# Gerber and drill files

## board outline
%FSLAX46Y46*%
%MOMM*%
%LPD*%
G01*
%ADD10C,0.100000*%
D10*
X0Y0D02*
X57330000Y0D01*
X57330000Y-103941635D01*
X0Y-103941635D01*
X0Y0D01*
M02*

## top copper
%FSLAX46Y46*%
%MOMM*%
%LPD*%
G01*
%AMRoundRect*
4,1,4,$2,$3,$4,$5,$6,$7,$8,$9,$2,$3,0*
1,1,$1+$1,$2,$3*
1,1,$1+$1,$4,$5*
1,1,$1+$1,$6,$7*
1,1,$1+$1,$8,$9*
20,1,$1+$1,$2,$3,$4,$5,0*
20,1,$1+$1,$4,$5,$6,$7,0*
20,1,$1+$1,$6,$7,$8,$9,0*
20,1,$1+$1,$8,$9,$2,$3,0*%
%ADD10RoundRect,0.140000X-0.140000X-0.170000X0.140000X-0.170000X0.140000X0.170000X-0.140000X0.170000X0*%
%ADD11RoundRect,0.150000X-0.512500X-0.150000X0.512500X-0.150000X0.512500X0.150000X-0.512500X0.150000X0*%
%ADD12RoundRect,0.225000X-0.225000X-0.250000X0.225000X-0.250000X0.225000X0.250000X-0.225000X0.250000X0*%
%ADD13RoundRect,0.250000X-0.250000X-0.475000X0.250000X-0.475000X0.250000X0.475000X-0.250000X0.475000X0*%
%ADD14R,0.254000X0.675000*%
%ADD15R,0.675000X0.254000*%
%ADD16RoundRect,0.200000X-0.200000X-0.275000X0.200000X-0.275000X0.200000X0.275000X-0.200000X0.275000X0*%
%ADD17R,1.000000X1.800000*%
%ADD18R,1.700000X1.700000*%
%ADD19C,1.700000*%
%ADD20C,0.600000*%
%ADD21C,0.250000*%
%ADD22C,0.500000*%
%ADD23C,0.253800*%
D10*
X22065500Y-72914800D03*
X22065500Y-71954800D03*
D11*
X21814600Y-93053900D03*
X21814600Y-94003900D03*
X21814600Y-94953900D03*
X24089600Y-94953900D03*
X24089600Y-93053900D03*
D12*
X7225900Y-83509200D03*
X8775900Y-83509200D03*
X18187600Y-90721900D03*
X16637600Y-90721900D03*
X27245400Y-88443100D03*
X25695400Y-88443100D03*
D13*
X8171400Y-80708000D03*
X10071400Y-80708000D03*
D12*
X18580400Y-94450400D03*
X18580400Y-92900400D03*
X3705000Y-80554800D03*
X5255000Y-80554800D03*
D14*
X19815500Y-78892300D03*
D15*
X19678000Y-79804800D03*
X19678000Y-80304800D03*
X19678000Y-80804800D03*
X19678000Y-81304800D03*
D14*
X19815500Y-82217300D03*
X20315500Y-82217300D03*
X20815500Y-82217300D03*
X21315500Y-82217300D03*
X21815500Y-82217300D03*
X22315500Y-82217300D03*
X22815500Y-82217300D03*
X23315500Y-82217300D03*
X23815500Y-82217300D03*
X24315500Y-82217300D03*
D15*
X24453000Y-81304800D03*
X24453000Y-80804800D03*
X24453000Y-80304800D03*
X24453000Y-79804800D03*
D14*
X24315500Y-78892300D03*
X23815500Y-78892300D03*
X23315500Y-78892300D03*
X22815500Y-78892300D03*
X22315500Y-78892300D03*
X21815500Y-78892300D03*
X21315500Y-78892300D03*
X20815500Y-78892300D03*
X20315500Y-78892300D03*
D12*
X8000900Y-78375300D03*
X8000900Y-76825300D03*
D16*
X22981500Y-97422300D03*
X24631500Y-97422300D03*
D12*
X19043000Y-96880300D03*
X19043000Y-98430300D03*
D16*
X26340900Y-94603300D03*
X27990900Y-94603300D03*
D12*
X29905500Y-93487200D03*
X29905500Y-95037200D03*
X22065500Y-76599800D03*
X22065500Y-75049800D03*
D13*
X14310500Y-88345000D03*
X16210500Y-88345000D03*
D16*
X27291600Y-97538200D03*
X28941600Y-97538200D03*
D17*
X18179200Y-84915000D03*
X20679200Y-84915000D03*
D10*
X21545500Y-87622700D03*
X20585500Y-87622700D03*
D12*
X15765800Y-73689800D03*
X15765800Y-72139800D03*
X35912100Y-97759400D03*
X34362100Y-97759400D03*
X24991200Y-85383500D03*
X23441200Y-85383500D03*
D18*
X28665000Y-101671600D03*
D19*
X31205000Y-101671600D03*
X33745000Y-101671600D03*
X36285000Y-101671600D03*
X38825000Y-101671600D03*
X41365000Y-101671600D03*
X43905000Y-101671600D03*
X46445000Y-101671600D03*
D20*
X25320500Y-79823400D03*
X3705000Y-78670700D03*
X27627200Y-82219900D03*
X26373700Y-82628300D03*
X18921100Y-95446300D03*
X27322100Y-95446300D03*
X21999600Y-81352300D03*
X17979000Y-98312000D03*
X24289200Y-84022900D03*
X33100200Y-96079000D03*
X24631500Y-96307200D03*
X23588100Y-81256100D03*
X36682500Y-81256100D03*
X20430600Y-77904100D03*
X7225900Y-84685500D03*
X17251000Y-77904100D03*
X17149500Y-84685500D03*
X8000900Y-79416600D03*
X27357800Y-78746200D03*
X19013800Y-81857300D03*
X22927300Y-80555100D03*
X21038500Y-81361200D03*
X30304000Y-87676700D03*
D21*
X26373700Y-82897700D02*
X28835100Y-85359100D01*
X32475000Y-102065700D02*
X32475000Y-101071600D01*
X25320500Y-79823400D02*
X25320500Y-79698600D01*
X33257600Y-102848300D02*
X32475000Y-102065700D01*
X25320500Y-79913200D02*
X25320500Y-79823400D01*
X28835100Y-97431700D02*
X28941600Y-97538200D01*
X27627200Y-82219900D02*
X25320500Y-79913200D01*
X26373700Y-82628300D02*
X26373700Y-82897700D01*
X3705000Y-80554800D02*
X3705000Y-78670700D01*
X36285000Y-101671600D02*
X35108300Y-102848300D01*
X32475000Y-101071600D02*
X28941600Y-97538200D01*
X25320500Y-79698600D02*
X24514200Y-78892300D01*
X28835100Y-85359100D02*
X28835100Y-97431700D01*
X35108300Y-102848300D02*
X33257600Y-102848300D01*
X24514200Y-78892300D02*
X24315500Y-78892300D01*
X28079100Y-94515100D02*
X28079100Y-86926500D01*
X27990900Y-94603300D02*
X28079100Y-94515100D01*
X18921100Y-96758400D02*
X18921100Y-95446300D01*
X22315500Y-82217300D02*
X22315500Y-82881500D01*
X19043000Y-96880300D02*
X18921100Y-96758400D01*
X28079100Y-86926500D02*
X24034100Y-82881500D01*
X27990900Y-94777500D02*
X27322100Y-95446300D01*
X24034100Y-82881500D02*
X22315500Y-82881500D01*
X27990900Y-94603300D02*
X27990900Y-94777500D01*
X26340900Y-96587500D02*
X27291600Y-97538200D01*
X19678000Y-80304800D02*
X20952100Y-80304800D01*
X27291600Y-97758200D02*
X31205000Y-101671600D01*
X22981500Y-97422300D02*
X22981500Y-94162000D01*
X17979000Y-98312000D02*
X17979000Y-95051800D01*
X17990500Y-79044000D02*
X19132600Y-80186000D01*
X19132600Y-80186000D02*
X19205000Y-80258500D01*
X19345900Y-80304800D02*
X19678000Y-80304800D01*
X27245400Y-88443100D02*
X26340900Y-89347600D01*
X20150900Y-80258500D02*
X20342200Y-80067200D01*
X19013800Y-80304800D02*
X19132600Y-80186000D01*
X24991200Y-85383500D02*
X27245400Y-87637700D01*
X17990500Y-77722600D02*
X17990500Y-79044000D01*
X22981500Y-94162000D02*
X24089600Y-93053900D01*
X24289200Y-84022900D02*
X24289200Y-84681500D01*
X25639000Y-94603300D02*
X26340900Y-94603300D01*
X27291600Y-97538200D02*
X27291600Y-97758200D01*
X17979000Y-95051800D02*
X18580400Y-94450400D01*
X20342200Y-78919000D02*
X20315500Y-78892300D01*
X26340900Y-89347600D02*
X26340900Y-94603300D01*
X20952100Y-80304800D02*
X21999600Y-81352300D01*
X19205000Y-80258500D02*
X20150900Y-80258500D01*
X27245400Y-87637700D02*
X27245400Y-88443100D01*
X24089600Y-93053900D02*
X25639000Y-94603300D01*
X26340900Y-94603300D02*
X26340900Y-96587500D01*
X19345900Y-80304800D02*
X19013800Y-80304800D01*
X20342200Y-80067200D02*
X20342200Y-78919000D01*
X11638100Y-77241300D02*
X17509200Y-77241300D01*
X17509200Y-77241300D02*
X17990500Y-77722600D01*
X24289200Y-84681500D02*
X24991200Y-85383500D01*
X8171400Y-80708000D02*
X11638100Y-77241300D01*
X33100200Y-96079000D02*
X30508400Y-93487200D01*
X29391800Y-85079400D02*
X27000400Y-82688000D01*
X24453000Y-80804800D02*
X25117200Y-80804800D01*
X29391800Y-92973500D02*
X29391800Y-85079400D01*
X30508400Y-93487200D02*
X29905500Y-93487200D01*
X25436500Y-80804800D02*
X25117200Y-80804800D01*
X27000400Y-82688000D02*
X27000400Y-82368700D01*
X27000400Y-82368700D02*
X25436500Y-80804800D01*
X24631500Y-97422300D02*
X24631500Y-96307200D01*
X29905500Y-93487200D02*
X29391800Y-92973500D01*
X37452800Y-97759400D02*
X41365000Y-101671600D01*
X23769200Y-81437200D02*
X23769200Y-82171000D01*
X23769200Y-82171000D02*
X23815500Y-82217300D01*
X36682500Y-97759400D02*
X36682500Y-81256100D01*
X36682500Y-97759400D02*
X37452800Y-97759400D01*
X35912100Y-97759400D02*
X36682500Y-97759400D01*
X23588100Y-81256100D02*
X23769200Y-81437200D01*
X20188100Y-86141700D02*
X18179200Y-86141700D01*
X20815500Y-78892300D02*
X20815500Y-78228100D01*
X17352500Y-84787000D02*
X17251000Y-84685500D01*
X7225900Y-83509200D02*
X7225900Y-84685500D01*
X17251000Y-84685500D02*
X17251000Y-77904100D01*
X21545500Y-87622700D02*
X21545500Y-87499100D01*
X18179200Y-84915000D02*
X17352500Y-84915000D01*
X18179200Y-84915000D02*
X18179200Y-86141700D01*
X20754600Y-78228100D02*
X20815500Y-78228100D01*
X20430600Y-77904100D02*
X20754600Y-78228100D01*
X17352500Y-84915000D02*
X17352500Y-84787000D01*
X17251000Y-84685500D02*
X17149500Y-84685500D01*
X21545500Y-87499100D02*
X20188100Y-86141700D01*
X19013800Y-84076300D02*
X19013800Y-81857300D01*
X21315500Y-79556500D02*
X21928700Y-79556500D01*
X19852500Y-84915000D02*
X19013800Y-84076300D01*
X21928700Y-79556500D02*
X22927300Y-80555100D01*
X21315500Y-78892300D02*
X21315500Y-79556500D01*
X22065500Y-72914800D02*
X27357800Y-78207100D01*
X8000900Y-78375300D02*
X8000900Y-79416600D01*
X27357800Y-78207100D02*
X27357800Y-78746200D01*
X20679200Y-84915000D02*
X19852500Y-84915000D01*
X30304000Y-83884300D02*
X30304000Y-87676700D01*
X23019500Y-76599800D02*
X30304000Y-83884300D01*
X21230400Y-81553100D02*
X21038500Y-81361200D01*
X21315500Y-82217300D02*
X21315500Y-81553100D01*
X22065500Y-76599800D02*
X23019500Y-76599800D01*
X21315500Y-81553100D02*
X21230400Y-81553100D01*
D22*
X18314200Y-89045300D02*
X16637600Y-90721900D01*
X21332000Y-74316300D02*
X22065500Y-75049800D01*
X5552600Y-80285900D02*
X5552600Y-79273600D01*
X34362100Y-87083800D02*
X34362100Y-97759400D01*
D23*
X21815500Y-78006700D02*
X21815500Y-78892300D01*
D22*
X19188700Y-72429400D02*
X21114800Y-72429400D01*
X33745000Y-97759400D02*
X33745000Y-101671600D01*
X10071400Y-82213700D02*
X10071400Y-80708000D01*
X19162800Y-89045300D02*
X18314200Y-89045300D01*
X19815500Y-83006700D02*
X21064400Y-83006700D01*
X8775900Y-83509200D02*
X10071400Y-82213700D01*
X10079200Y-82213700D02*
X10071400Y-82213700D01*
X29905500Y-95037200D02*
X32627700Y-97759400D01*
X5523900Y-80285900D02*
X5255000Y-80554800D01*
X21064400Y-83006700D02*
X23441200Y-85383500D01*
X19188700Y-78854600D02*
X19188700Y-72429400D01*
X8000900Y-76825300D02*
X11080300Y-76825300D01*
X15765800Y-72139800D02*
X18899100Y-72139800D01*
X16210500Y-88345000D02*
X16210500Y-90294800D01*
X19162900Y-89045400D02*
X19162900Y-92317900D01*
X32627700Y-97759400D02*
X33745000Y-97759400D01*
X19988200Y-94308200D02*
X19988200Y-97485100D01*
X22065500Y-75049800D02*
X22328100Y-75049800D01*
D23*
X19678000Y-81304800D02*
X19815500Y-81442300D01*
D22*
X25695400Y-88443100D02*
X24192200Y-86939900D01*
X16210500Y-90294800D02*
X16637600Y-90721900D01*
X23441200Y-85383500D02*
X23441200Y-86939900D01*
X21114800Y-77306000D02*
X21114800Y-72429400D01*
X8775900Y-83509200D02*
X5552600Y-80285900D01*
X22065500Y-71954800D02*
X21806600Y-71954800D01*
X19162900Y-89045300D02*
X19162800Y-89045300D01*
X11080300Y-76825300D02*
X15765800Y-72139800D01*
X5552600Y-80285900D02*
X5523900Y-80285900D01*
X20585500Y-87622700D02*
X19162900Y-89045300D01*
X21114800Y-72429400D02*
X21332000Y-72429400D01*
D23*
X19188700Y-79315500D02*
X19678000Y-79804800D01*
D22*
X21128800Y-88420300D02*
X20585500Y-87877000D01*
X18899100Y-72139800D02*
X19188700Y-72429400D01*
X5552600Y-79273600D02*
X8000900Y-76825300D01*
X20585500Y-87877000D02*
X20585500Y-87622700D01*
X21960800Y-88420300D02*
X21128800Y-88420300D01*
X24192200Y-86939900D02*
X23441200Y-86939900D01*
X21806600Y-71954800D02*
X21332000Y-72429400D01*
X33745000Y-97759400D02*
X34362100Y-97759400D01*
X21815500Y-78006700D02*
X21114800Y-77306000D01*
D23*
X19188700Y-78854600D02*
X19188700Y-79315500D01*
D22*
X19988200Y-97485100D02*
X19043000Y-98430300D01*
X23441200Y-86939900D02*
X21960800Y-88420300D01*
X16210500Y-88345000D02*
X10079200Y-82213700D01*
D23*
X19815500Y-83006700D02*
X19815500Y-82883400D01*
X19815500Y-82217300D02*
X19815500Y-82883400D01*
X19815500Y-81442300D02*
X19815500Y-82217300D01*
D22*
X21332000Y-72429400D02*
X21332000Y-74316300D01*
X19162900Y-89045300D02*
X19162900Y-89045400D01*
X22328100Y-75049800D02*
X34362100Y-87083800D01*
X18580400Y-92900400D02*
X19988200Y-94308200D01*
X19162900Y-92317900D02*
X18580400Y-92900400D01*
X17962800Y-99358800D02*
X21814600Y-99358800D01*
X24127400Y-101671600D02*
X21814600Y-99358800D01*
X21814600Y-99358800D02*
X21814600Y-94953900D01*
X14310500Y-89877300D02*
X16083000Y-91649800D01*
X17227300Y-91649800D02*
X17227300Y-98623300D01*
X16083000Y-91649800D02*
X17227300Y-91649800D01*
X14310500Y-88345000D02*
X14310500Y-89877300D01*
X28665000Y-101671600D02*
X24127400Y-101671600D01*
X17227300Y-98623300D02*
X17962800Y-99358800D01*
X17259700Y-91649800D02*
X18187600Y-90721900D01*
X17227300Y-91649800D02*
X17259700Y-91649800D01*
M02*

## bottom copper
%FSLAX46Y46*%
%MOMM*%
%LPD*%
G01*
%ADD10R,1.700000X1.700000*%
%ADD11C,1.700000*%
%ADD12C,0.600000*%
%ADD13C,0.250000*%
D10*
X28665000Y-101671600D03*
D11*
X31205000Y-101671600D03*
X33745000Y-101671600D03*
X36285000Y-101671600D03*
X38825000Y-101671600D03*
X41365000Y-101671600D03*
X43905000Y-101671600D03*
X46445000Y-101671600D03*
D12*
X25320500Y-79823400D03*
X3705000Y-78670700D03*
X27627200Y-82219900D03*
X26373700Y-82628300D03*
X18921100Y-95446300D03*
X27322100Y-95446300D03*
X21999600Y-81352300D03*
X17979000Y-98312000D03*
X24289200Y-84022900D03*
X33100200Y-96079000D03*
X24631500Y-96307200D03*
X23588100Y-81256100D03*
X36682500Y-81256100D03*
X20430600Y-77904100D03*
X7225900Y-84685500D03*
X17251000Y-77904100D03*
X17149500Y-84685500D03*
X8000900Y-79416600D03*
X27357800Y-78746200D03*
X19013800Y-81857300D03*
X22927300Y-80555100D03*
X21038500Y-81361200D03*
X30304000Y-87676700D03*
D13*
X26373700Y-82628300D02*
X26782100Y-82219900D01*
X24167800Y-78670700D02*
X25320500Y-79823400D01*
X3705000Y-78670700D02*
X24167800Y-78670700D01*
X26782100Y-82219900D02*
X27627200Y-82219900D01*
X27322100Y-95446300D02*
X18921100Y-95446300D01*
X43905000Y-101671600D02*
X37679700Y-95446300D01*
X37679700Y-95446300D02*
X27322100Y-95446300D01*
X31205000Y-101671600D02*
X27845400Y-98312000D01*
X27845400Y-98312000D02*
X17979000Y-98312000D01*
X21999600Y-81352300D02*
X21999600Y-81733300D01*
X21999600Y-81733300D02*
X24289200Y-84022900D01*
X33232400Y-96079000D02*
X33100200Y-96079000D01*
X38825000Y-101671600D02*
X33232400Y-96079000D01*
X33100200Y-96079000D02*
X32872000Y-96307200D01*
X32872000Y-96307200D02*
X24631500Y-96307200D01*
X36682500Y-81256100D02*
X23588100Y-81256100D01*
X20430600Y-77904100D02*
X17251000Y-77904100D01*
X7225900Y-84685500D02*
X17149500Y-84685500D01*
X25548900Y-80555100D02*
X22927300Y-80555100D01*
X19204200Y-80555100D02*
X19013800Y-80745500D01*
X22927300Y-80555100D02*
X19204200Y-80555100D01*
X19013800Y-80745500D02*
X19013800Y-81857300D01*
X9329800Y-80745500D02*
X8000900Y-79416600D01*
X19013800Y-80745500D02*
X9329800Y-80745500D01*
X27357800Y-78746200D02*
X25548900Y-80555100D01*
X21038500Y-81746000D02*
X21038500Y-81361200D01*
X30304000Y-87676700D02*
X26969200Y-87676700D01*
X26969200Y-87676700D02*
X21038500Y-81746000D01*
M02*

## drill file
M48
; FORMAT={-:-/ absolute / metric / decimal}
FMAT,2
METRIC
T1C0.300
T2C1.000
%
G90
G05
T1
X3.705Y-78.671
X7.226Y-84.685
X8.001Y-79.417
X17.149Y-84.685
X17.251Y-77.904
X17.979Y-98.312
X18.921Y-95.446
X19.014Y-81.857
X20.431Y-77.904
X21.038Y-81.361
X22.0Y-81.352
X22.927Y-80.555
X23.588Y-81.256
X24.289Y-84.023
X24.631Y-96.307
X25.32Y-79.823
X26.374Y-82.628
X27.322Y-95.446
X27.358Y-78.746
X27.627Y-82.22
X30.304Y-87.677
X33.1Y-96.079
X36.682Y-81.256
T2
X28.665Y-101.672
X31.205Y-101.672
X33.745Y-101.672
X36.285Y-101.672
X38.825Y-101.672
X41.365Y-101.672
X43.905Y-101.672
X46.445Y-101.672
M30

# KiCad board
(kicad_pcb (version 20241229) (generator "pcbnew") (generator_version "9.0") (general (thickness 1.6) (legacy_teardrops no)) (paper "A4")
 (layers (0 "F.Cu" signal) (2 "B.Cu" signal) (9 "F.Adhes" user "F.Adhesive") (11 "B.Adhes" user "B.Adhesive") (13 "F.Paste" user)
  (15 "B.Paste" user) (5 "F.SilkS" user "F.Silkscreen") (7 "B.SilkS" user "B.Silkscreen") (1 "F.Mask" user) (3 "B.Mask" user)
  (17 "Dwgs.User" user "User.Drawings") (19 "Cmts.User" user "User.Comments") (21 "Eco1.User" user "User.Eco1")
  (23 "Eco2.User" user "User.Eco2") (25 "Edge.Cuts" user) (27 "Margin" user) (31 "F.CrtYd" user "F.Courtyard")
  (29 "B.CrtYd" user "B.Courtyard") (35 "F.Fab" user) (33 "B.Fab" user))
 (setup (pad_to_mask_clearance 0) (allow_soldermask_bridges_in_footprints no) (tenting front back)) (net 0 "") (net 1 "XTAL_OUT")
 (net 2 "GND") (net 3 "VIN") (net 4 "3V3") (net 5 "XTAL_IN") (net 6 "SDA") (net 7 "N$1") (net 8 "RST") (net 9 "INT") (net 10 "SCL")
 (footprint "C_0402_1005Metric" (layer "F.Cu") (at 22.0655 72.4348 90)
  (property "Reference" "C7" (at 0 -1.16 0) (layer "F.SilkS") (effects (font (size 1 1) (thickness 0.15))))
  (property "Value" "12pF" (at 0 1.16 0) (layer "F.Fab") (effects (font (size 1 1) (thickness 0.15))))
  (pad "1" smd roundrect (at -0.48 0) (size 0.56 0.62) (layers "F.Cu" "F.Mask" "F.Paste") (roundrect_rratio 0.25) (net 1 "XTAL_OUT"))
  (pad "2" smd roundrect (at 0.48 0) (size 0.56 0.62) (layers "F.Cu" "F.Mask" "F.Paste") (roundrect_rratio 0.25) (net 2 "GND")))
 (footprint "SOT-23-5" (layer "F.Cu") (at 22.9521 94.0039)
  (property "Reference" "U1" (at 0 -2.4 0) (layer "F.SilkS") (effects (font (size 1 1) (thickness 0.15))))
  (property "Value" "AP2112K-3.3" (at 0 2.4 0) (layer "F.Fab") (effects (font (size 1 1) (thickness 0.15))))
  (pad "1" smd roundrect (at -1.1375 -0.95) (size 1.325 0.6) (layers "F.Cu" "F.Mask" "F.Paste") (roundrect_rratio 0.25) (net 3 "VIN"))
  (pad "2" smd roundrect (at -1.1375 0) (size 1.325 0.6) (layers "F.Cu" "F.Mask" "F.Paste") (roundrect_rratio 0.25) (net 2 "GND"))
  (pad "3" smd roundrect (at -1.1375 0.95) (size 1.325 0.6) (layers "F.Cu" "F.Mask" "F.Paste") (roundrect_rratio 0.25) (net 3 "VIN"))
  (pad "4" smd roundrect (at 1.1375 0.95) (size 1.325 0.6) (layers "F.Cu" "F.Mask" "F.Paste") (roundrect_rratio 0.25))
  (pad "5" smd roundrect (at 1.1375 -0.95) (size 1.325 0.6) (layers "F.Cu" "F.Mask" "F.Paste") (roundrect_rratio 0.25) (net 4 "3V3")))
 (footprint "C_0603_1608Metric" (layer "F.Cu") (at 8.0009 83.5092)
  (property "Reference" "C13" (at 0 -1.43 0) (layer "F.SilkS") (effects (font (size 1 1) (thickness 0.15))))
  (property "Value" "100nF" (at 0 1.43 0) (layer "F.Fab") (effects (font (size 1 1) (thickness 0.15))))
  (pad "1" smd roundrect (at -0.775 0) (size 0.9 0.95) (layers "F.Cu" "F.Mask" "F.Paste") (roundrect_rratio 0.25) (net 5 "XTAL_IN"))
  (pad "2" smd roundrect (at 0.775 0) (size 0.9 0.95) (layers "F.Cu" "F.Mask" "F.Paste") (roundrect_rratio 0.25) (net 2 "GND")))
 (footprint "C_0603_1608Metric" (layer "F.Cu") (at 17.4126 90.7219 180)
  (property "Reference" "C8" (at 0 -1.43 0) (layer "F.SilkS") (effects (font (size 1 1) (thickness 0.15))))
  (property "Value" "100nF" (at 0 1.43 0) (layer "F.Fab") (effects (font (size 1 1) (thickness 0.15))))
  (pad "1" smd roundrect (at -0.775 0) (size 0.9 0.95) (layers "F.Cu" "F.Mask" "F.Paste") (roundrect_rratio 0.25) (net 3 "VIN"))
  (pad "2" smd roundrect (at 0.775 0) (size 0.9 0.95) (layers "F.Cu" "F.Mask" "F.Paste") (roundrect_rratio 0.25) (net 2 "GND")))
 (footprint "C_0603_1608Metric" (layer "F.Cu") (at 26.4704 88.4431 180)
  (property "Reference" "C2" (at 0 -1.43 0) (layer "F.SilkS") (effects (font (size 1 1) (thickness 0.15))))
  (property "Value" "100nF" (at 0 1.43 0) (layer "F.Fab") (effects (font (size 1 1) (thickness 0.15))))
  (pad "1" smd roundrect (at -0.775 0) (size 0.9 0.95) (layers "F.Cu" "F.Mask" "F.Paste") (roundrect_rratio 0.25) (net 4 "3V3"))
  (pad "2" smd roundrect (at 0.775 0) (size 0.9 0.95) (layers "F.Cu" "F.Mask" "F.Paste") (roundrect_rratio 0.25) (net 2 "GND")))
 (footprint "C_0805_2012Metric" (layer "F.Cu") (at 9.1214 80.708)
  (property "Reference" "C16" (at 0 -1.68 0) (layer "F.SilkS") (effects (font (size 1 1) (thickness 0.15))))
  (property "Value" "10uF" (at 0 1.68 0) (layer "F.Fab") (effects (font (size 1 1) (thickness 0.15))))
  (pad "1" smd roundrect (at -0.95 0) (size 1 1.45) (layers "F.Cu" "F.Mask" "F.Paste") (roundrect_rratio 0.25) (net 4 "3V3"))
  (pad "2" smd roundrect (at 0.95 0) (size 1 1.45) (layers "F.Cu" "F.Mask" "F.Paste") (roundrect_rratio 0.25) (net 2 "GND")))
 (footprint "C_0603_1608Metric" (layer "F.Cu") (at 18.5804 93.6754 90)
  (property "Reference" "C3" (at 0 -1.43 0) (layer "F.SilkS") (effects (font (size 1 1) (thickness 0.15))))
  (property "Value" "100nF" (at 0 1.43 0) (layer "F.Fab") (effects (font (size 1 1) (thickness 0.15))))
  (pad "1" smd roundrect (at -0.775 0) (size 0.9 0.95) (layers "F.Cu" "F.Mask" "F.Paste") (roundrect_rratio 0.25) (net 4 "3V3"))
  (pad "2" smd roundrect (at 0.775 0) (size 0.9 0.95) (layers "F.Cu" "F.Mask" "F.Paste") (roundrect_rratio 0.25) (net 2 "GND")))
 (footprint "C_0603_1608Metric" (layer "F.Cu") (at 4.48 80.5548)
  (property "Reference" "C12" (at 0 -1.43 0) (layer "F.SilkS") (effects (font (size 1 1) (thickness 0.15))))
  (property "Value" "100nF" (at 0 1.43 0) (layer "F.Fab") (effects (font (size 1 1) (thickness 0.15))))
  (pad "1" smd roundrect (at -0.775 0) (size 0.9 0.95) (layers "F.Cu" "F.Mask" "F.Paste") (roundrect_rratio 0.25) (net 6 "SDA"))
  (pad "2" smd roundrect (at 0.775 0) (size 0.9 0.95) (layers "F.Cu" "F.Mask" "F.Paste") (roundrect_rratio 0.25) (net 2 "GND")))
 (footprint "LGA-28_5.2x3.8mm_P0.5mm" (layer "F.Cu") (at 22.0655 80.5548)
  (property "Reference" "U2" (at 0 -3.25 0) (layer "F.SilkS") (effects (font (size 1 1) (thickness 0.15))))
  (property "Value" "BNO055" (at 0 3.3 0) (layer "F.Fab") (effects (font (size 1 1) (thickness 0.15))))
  (pad "1" smd rect (at -2.25 -1.6625) (size 0.254 0.675) (layers "F.Cu" "F.Mask" "F.Paste"))
  (pad "2" smd rect (at -2.3875 -0.75 90) (size 0.254 0.675) (layers "F.Cu" "F.Mask" "F.Paste") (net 2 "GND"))
  (pad "3" smd rect (at -2.3875 -0.25 90) (size 0.254 0.675) (layers "F.Cu" "F.Mask" "F.Paste") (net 4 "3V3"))
  (pad "4" smd rect (at -2.3875 0.25 90) (size 0.254 0.675) (layers "F.Cu" "F.Mask" "F.Paste"))
  (pad "5" smd rect (at -2.3875 0.75 90) (size 0.254 0.675) (layers "F.Cu" "F.Mask" "F.Paste") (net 2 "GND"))
  (pad "6" smd rect (at -2.25 1.6625) (size 0.254 0.675) (layers "F.Cu" "F.Mask" "F.Paste") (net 2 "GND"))
  (pad "7" smd rect (at -1.75 1.6625) (size 0.254 0.675) (layers "F.Cu" "F.Mask" "F.Paste"))
  (pad "8" smd rect (at -1.25 1.6625) (size 0.254 0.675) (layers "F.Cu" "F.Mask" "F.Paste"))
  (pad "9" smd rect (at -0.75 1.6625) (size 0.254 0.675) (layers "F.Cu" "F.Mask" "F.Paste") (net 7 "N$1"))
  (pad "10" smd rect (at -0.25 1.6625) (size 0.254 0.675) (layers "F.Cu" "F.Mask" "F.Paste"))
  (pad "11" smd rect (at 0.25 1.6625) (size 0.254 0.675) (layers "F.Cu" "F.Mask" "F.Paste") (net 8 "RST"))
  (pad "12" smd rect (at 0.75 1.6625) (size 0.254 0.675) (layers "F.Cu" "F.Mask" "F.Paste"))
  (pad "13" smd rect (at 1.25 1.6625) (size 0.254 0.675) (layers "F.Cu" "F.Mask" "F.Paste"))
  (pad "14" smd rect (at 1.75 1.6625) (size 0.254 0.675) (layers "F.Cu" "F.Mask" "F.Paste") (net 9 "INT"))
  (pad "15" smd rect (at 2.25 1.6625) (size 0.254 0.675) (layers "F.Cu" "F.Mask" "F.Paste"))
  (pad "16" smd rect (at 2.3875 0.75 90) (size 0.254 0.675) (layers "F.Cu" "F.Mask" "F.Paste"))
  (pad "17" smd rect (at 2.3875 0.25 90) (size 0.254 0.675) (layers "F.Cu" "F.Mask" "F.Paste") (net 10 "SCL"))
  (pad "18" smd rect (at 2.3875 -0.25 90) (size 0.254 0.675) (layers "F.Cu" "F.Mask" "F.Paste"))
  (pad "19" smd rect (at 2.3875 -0.75 90) (size 0.254 0.675) (layers "F.Cu" "F.Mask" "F.Paste"))
  (pad "20" smd rect (at 2.25 -1.6625) (size 0.254 0.675) (layers "F.Cu" "F.Mask" "F.Paste") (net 6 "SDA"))
  (pad "21" smd rect (at 1.75 -1.6625) (size 0.254 0.675) (layers "F.Cu" "F.Mask" "F.Paste"))
  (pad "22" smd rect (at 1.25 -1.6625) (size 0.254 0.675) (layers "F.Cu" "F.Mask" "F.Paste"))
  (pad "23" smd rect (at 0.75 -1.6625) (size 0.254 0.675) (layers "F.Cu" "F.Mask" "F.Paste"))
  (pad "24" smd rect (at 0.25 -1.6625) (size 0.254 0.675) (layers "F.Cu" "F.Mask" "F.Paste"))
  (pad "25" smd rect (at -0.25 -1.6625) (size 0.254 0.675) (layers "F.Cu" "F.Mask" "F.Paste") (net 2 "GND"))
  (pad "26" smd rect (at -0.75 -1.6625) (size 0.254 0.675) (layers "F.Cu" "F.Mask" "F.Paste") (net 1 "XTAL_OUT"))
  (pad "27" smd rect (at -1.25 -1.6625) (size 0.254 0.675) (layers "F.Cu" "F.Mask" "F.Paste") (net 5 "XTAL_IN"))
  (pad "28" smd rect (at -1.75 -1.6625) (size 0.254 0.675) (layers "F.Cu" "F.Mask" "F.Paste") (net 4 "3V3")))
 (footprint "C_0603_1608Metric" (layer "F.Cu") (at 8.0009 77.6003 90)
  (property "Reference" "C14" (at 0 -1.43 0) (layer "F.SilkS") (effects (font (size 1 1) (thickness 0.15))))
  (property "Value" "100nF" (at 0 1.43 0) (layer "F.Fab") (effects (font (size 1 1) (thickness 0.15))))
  (pad "1" smd roundrect (at -0.775 0) (size 0.9 0.95) (layers "F.Cu" "F.Mask" "F.Paste") (roundrect_rratio 0.25) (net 1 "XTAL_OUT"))
  (pad "2" smd roundrect (at 0.775 0) (size 0.9 0.95) (layers "F.Cu" "F.Mask" "F.Paste") (roundrect_rratio 0.25) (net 2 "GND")))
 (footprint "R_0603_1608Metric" (layer "F.Cu") (at 23.8065 97.4223)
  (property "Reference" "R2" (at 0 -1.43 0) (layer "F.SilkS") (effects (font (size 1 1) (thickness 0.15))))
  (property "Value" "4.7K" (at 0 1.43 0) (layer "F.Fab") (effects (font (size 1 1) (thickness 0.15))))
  (pad "1" smd roundrect (at -0.825 0) (size 0.8 0.95) (layers "F.Cu" "F.Mask" "F.Paste") (roundrect_rratio 0.25) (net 4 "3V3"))
  (pad "2" smd roundrect (at 0.825 0) (size 0.8 0.95) (layers "F.Cu" "F.Mask" "F.Paste") (roundrect_rratio 0.25) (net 10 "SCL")))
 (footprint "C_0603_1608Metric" (layer "F.Cu") (at 19.043 97.6553 -90)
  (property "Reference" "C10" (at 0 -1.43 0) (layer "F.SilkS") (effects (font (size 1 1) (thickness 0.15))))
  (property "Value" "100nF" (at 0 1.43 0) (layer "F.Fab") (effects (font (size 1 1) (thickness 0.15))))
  (pad "1" smd roundrect (at -0.775 0) (size 0.9 0.95) (layers "F.Cu" "F.Mask" "F.Paste") (roundrect_rratio 0.25) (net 8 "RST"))
  (pad "2" smd roundrect (at 0.775 0) (size 0.9 0.95) (layers "F.Cu" "F.Mask" "F.Paste") (roundrect_rratio 0.25) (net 2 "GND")))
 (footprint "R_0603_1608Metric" (layer "F.Cu") (at 27.1659 94.6033)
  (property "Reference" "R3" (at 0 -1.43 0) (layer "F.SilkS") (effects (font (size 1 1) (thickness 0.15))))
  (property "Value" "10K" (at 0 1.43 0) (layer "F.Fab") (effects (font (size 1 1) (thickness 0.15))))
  (pad "1" smd roundrect (at -0.825 0) (size 0.8 0.95) (layers "F.Cu" "F.Mask" "F.Paste") (roundrect_rratio 0.25) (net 4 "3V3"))
  (pad "2" smd roundrect (at 0.825 0) (size 0.8 0.95) (layers "F.Cu" "F.Mask" "F.Paste") (roundrect_rratio 0.25) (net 8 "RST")))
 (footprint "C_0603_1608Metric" (layer "F.Cu") (at 29.9055 94.2622 -90)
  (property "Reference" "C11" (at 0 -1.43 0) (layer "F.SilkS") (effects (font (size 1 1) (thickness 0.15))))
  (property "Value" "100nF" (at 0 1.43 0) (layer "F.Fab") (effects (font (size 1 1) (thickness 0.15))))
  (pad "1" smd roundrect (at -0.775 0) (size 0.9 0.95) (layers "F.Cu" "F.Mask" "F.Paste") (roundrect_rratio 0.25) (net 10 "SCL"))
  (pad "2" smd roundrect (at 0.775 0) (size 0.9 0.95) (layers "F.Cu" "F.Mask" "F.Paste") (roundrect_rratio 0.25) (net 2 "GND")))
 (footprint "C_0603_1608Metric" (layer "F.Cu") (at 22.0655 75.8248 90)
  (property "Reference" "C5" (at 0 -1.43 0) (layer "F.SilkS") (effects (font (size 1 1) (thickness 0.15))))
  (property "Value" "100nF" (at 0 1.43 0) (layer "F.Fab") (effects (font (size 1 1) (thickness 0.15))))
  (pad "1" smd roundrect (at -0.775 0) (size 0.9 0.95) (layers "F.Cu" "F.Mask" "F.Paste") (roundrect_rratio 0.25) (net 7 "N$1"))
  (pad "2" smd roundrect (at 0.775 0) (size 0.9 0.95) (layers "F.Cu" "F.Mask" "F.Paste") (roundrect_rratio 0.25) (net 2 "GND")))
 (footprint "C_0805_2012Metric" (layer "F.Cu") (at 15.2605 88.345)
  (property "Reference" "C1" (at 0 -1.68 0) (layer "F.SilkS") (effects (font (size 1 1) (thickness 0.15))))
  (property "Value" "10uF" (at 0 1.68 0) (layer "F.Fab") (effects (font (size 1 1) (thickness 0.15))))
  (pad "1" smd roundrect (at -0.95 0) (size 1 1.45) (layers "F.Cu" "F.Mask" "F.Paste") (roundrect_rratio 0.25) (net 3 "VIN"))
  (pad "2" smd roundrect (at 0.95 0) (size 1 1.45) (layers "F.Cu" "F.Mask" "F.Paste") (roundrect_rratio 0.25) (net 2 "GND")))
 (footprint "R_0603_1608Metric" (layer "F.Cu") (at 28.1166 97.5382)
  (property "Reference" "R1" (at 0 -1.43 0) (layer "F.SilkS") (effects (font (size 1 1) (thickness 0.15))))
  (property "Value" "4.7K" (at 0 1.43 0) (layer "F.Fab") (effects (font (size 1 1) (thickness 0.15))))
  (pad "1" smd roundrect (at -0.825 0) (size 0.8 0.95) (layers "F.Cu" "F.Mask" "F.Paste") (roundrect_rratio 0.25) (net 4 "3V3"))
  (pad "2" smd roundrect (at 0.825 0) (size 0.8 0.95) (layers "F.Cu" "F.Mask" "F.Paste") (roundrect_rratio 0.25) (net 6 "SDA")))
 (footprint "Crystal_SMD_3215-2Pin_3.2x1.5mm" (layer "F.Cu") (at 19.4292 84.915 180)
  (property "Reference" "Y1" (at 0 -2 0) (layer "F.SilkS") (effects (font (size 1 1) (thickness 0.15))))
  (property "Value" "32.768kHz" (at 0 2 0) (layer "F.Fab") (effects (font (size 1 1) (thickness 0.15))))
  (pad "1" smd rect (at 1.25 0) (size 1 1.8) (layers "F.Cu" "F.Mask" "F.Paste") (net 5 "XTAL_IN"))
  (pad "2" smd rect (at -1.25 0) (size 1 1.8) (layers "F.Cu" "F.Mask" "F.Paste") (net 1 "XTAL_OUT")))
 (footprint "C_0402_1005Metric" (layer "F.Cu") (at 21.0655 87.6227 180)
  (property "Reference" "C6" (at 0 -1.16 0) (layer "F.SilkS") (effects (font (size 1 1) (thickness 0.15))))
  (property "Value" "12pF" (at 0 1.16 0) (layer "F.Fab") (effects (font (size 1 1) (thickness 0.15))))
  (pad "1" smd roundrect (at -0.48 0) (size 0.56 0.62) (layers "F.Cu" "F.Mask" "F.Paste") (roundrect_rratio 0.25) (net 5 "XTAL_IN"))
  (pad "2" smd roundrect (at 0.48 0) (size 0.56 0.62) (layers "F.Cu" "F.Mask" "F.Paste") (roundrect_rratio 0.25) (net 2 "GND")))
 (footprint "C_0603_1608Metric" (layer "F.Cu") (at 15.7658 72.9148 90)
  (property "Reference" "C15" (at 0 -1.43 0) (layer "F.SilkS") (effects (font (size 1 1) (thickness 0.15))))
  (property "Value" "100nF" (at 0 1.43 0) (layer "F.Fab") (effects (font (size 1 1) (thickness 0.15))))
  (pad "1" smd roundrect (at -0.775 0) (size 0.9 0.95) (layers "F.Cu" "F.Mask" "F.Paste") (roundrect_rratio 0.25))
  (pad "2" smd roundrect (at 0.775 0) (size 0.9 0.95) (layers "F.Cu" "F.Mask" "F.Paste") (roundrect_rratio 0.25) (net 2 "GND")))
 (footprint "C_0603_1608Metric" (layer "F.Cu") (at 35.1371 97.7594 180)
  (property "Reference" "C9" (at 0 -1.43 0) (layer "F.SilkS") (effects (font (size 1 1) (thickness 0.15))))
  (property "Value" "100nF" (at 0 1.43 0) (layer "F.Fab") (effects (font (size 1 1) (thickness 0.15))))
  (pad "1" smd roundrect (at -0.775 0) (size 0.9 0.95) (layers "F.Cu" "F.Mask" "F.Paste") (roundrect_rratio 0.25) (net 9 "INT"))
  (pad "2" smd roundrect (at 0.775 0) (size 0.9 0.95) (layers "F.Cu" "F.Mask" "F.Paste") (roundrect_rratio 0.25) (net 2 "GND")))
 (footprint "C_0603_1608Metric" (layer "F.Cu") (at 24.2162 85.3835 180)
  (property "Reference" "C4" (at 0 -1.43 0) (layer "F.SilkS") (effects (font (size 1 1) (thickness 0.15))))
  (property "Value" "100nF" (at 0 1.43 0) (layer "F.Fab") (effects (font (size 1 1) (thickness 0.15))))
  (pad "1" smd roundrect (at -0.775 0) (size 0.9 0.95) (layers "F.Cu" "F.Mask" "F.Paste") (roundrect_rratio 0.25) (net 4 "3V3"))
  (pad "2" smd roundrect (at 0.775 0) (size 0.9 0.95) (layers "F.Cu" "F.Mask" "F.Paste") (roundrect_rratio 0.25) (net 2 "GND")))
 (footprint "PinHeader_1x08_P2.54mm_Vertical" (layer "F.Cu") (at 28.665 101.6716 90)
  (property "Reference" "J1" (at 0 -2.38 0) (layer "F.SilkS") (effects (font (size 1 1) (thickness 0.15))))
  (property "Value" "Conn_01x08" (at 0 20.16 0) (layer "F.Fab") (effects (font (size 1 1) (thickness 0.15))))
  (pad "1" thru_hole rect (at 0 0) (size 1.7 1.7) (drill 1) (layers "*.Cu" "*.Mask") (remove_unused_layers no) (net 3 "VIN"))
  (pad "2" thru_hole circle (at 0 2.54) (size 1.7 1.7) (drill 1) (layers "*.Cu" "*.Mask") (remove_unused_layers no) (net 4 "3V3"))
  (pad "3" thru_hole circle (at 0 5.08) (size 1.7 1.7) (drill 1) (layers "*.Cu" "*.Mask") (remove_unused_layers no) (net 2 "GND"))
  (pad "4" thru_hole circle (at 0 7.62) (size 1.7 1.7) (drill 1) (layers "*.Cu" "*.Mask") (remove_unused_layers no) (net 6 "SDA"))
  (pad "5" thru_hole circle (at 0 10.16) (size 1.7 1.7) (drill 1) (layers "*.Cu" "*.Mask") (remove_unused_layers no) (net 10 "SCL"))
  (pad "6" thru_hole circle (at 0 12.7) (size 1.7 1.7) (drill 1) (layers "*.Cu" "*.Mask") (remove_unused_layers no) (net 9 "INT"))
  (pad "7" thru_hole circle (at 0 15.24) (size 1.7 1.7) (drill 1) (layers "*.Cu" "*.Mask") (remove_unused_layers no) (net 8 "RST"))
  (pad "8" thru_hole circle (at 0 17.78) (size 1.7 1.7) (drill 1) (layers "*.Cu" "*.Mask") (remove_unused_layers no) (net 2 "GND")))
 (gr_rect (start 0 0) (end 57.33 103.941635) (stroke (width 0.1) (type solid)) (fill no) (layer "Edge.Cuts"))
 (segment (start 26.3737 82.8977) (end 28.8351 85.3591) (width 0.25) (layer "F.Cu") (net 6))
 (segment (start 32.475 102.0657) (end 32.475 101.0716) (width 0.25) (layer "F.Cu") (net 6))
 (segment (start 25.3205 79.8234) (end 25.3205 79.6986) (width 0.25) (layer "F.Cu") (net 6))
 (segment (start 33.2576 102.8483) (end 32.475 102.0657) (width 0.25) (layer "F.Cu") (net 6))
 (segment (start 25.3205 79.9132) (end 25.3205 79.8234) (width 0.25) (layer "F.Cu") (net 6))
 (segment (start 28.8351 97.4317) (end 28.9416 97.5382) (width 0.25) (layer "F.Cu") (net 6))
 (segment (start 27.6272 82.2199) (end 25.3205 79.9132) (width 0.25) (layer "F.Cu") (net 6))
 (segment (start 26.3737 82.6283) (end 26.3737 82.8977) (width 0.25) (layer "F.Cu") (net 6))
 (segment (start 3.705 80.5548) (end 3.705 78.6707) (width 0.25) (layer "F.Cu") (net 6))
 (segment (start 36.285 101.6716) (end 35.1083 102.8483) (width 0.25) (layer "F.Cu") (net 6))
 (segment (start 32.475 101.0716) (end 28.9416 97.5382) (width 0.25) (layer "F.Cu") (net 6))
 (segment (start 25.3205 79.6986) (end 24.5142 78.8923) (width 0.25) (layer "F.Cu") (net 6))
 (segment (start 28.8351 85.3591) (end 28.8351 97.4317) (width 0.25) (layer "F.Cu") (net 6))
 (segment (start 35.1083 102.8483) (end 33.2576 102.8483) (width 0.25) (layer "F.Cu") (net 6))
 (segment (start 24.5142 78.8923) (end 24.3155 78.8923) (width 0.25) (layer "F.Cu") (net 6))
 (via (at 25.3205 79.8234) (size 0.6) (drill 0.3) (layers "F.Cu" "B.Cu") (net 6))
 (via (at 3.705 78.6707) (size 0.6) (drill 0.3) (layers "F.Cu" "B.Cu") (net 6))
 (via (at 27.6272 82.2199) (size 0.6) (drill 0.3) (layers "F.Cu" "B.Cu") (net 6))
 (via (at 26.3737 82.6283) (size 0.6) (drill 0.3) (layers "F.Cu" "B.Cu") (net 6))
 (segment (start 26.3737 82.6283) (end 26.7821 82.2199) (width 0.25) (layer "B.Cu") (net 6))
 (segment (start 24.1678 78.6707) (end 25.3205 79.8234) (width 0.25) (layer "B.Cu") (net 6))
 (segment (start 3.705 78.6707) (end 24.1678 78.6707) (width 0.25) (layer "B.Cu") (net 6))
 (segment (start 26.7821 82.2199) (end 27.6272 82.2199) (width 0.25) (layer "B.Cu") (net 6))
 (segment (start 28.0791 94.5151) (end 28.0791 86.9265) (width 0.25) (layer "F.Cu") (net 8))
 (segment (start 27.9909 94.6033) (end 28.0791 94.5151) (width 0.25) (layer "F.Cu") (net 8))
 (segment (start 18.9211 96.7584) (end 18.9211 95.4463) (width 0.25) (layer "F.Cu") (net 8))
 (segment (start 22.3155 82.2173) (end 22.3155 82.8815) (width 0.25) (layer "F.Cu") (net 8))
 (segment (start 19.043 96.8803) (end 18.9211 96.7584) (width 0.25) (layer "F.Cu") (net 8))
 (segment (start 28.0791 86.9265) (end 24.0341 82.8815) (width 0.25) (layer "F.Cu") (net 8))
 (segment (start 27.9909 94.7775) (end 27.3221 95.4463) (width 0.25) (layer "F.Cu") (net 8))
 (segment (start 24.0341 82.8815) (end 22.3155 82.8815) (width 0.25) (layer "F.Cu") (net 8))
 (segment (start 27.9909 94.6033) (end 27.9909 94.7775) (width 0.25) (layer "F.Cu") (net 8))
 (via (at 18.9211 95.4463) (size 0.6) (drill 0.3) (layers "F.Cu" "B.Cu") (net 8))
 (via (at 27.3221 95.4463) (size 0.6) (drill 0.3) (layers "F.Cu" "B.Cu") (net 8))
 (segment (start 27.3221 95.4463) (end 18.9211 95.4463) (width 0.25) (layer "B.Cu") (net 8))
 (segment (start 43.905 101.6716) (end 37.6797 95.4463) (width 0.25) (layer "B.Cu") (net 8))
 (segment (start 37.6797 95.4463) (end 27.3221 95.4463) (width 0.25) (layer "B.Cu") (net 8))
 (segment (start 26.3409 96.5875) (end 27.2916 97.5382) (width 0.25) (layer "F.Cu") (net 4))
 (segment (start 19.678 80.3048) (end 20.9521 80.3048) (width 0.25) (layer "F.Cu") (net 4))
 (segment (start 27.2916 97.7582) (end 31.205 101.6716) (width 0.25) (layer "F.Cu") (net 4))
 (segment (start 22.9815 97.4223) (end 22.9815 94.162) (width 0.25) (layer "F.Cu") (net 4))
 (segment (start 17.979 98.312) (end 17.979 95.0518) (width 0.25) (layer "F.Cu") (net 4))
 (segment (start 17.9905 79.044) (end 19.1326 80.186) (width 0.25) (layer "F.Cu") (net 4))
 (segment (start 19.1326 80.186) (end 19.205 80.2585) (width 0.25) (layer "F.Cu") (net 4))
 (segment (start 19.3459 80.3048) (end 19.678 80.3048) (width 0.25) (layer "F.Cu") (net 4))
 (segment (start 27.2454 88.4431) (end 26.3409 89.3476) (width 0.25) (layer "F.Cu") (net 4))
 (segment (start 20.1509 80.2585) (end 20.3422 80.0672) (width 0.25) (layer "F.Cu") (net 4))
 (segment (start 19.0138 80.3048) (end 19.1326 80.186) (width 0.25) (layer "F.Cu") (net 4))
 (segment (start 24.9912 85.3835) (end 27.2454 87.6377) (width 0.25) (layer "F.Cu") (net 4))
 (segment (start 17.9905 77.7226) (end 17.9905 79.044) (width 0.25) (layer "F.Cu") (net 4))
 (segment (start 22.9815 94.162) (end 24.0896 93.0539) (width 0.25) (layer "F.Cu") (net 4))
 (segment (start 24.2892 84.0229) (end 24.2892 84.6815) (width 0.25) (layer "F.Cu") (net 4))
 (segment (start 25.639 94.6033) (end 26.3409 94.6033) (width 0.25) (layer "F.Cu") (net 4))
 (segment (start 27.2916 97.5382) (end 27.2916 97.7582) (width 0.25) (layer "F.Cu") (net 4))
 (segment (start 17.979 95.0518) (end 18.5804 94.4504) (width 0.25) (layer "F.Cu") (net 4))
 (segment (start 20.3422 78.919) (end 20.3155 78.8923) (width 0.25) (layer "F.Cu") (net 4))
 (segment (start 26.3409 89.3476) (end 26.3409 94.6033) (width 0.25) (layer "F.Cu") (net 4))
 (segment (start 20.9521 80.3048) (end 21.9996 81.3523) (width 0.25) (layer "F.Cu") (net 4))
 (segment (start 19.205 80.2585) (end 20.1509 80.2585) (width 0.25) (layer "F.Cu") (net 4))
 (segment (start 27.2454 87.6377) (end 27.2454 88.4431) (width 0.25) (layer "F.Cu") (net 4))
 (segment (start 24.0896 93.0539) (end 25.639 94.6033) (width 0.25) (layer "F.Cu") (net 4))
 (segment (start 26.3409 94.6033) (end 26.3409 96.5875) (width 0.25) (layer "F.Cu") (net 4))
 (segment (start 19.3459 80.3048) (end 19.0138 80.3048) (width 0.25) (layer "F.Cu") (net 4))
 (segment (start 20.3422 80.0672) (end 20.3422 78.919) (width 0.25) (layer "F.Cu") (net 4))
 (segment (start 11.6381 77.2413) (end 17.5092 77.2413) (width 0.25) (layer "F.Cu") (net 4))
 (segment (start 17.5092 77.2413) (end 17.9905 77.7226) (width 0.25) (layer "F.Cu") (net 4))
 (segment (start 24.2892 84.6815) (end 24.9912 85.3835) (width 0.25) (layer "F.Cu") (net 4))
 (segment (start 8.1714 80.708) (end 11.6381 77.2413) (width 0.25) (layer "F.Cu") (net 4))
 (via (at 21.9996 81.3523) (size 0.6) (drill 0.3) (layers "F.Cu" "B.Cu") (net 4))
 (via (at 17.979 98.312) (size 0.6) (drill 0.3) (layers "F.Cu" "B.Cu") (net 4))
 (via (at 24.2892 84.0229) (size 0.6) (drill 0.3) (layers "F.Cu" "B.Cu") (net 4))
 (segment (start 31.205 101.6716) (end 27.8454 98.312) (width 0.25) (layer "B.Cu") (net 4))
 (segment (start 27.8454 98.312) (end 17.979 98.312) (width 0.25) (layer "B.Cu") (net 4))
 (segment (start 21.9996 81.3523) (end 21.9996 81.7333) (width 0.25) (layer "B.Cu") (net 4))
 (segment (start 21.9996 81.7333) (end 24.2892 84.0229) (width 0.25) (layer "B.Cu") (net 4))
 (segment (start 33.1002 96.079) (end 30.5084 93.4872) (width 0.25) (layer "F.Cu") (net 10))
 (segment (start 29.3918 85.0794) (end 27.0004 82.688) (width 0.25) (layer "F.Cu") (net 10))
 (segment (start 24.453 80.8048) (end 25.1172 80.8048) (width 0.25) (layer "F.Cu") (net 10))
 (segment (start 29.3918 92.9735) (end 29.3918 85.0794) (width 0.25) (layer "F.Cu") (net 10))
 (segment (start 30.5084 93.4872) (end 29.9055 93.4872) (width 0.25) (layer "F.Cu") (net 10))
 (segment (start 25.4365 80.8048) (end 25.1172 80.8048) (width 0.25) (layer "F.Cu") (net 10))
 (segment (start 27.0004 82.688) (end 27.0004 82.3687) (width 0.25) (layer "F.Cu") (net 10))
 (segment (start 27.0004 82.3687) (end 25.4365 80.8048) (width 0.25) (layer "F.Cu") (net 10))
 (segment (start 24.6315 97.4223) (end 24.6315 96.3072) (width 0.25) (layer "F.Cu") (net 10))
 (segment (start 29.9055 93.4872) (end 29.3918 92.9735) (width 0.25) (layer "F.Cu") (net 10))
 (via (at 33.1002 96.079) (size 0.6) (drill 0.3) (layers "F.Cu" "B.Cu") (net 10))
 (via (at 24.6315 96.3072) (size 0.6) (drill 0.3) (layers "F.Cu" "B.Cu") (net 10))
 (segment (start 33.2324 96.079) (end 33.1002 96.079) (width 0.25) (layer "B.Cu") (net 10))
 (segment (start 38.825 101.6716) (end 33.2324 96.079) (width 0.25) (layer "B.Cu") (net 10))
 (segment (start 33.1002 96.079) (end 32.872 96.3072) (width 0.25) (layer "B.Cu") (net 10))
 (segment (start 32.872 96.3072) (end 24.6315 96.3072) (width 0.25) (layer "B.Cu") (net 10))
 (segment (start 37.4528 97.7594) (end 41.365 101.6716) (width 0.25) (layer "F.Cu") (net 9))
 (segment (start 23.7692 81.4372) (end 23.7692 82.171) (width 0.25) (layer "F.Cu") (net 9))
 (segment (start 23.7692 82.171) (end 23.8155 82.2173) (width 0.25) (layer "F.Cu") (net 9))
 (segment (start 36.6825 97.7594) (end 36.6825 81.2561) (width 0.25) (layer "F.Cu") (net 9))
 (segment (start 36.6825 97.7594) (end 37.4528 97.7594) (width 0.25) (layer "F.Cu") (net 9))
 (segment (start 35.9121 97.7594) (end 36.6825 97.7594) (width 0.25) (layer "F.Cu") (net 9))
 (segment (start 23.5881 81.2561) (end 23.7692 81.4372) (width 0.25) (layer "F.Cu") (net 9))
 (via (at 23.5881 81.2561) (size 0.6) (drill 0.3) (layers "F.Cu" "B.Cu") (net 9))
 (via (at 36.6825 81.2561) (size 0.6) (drill 0.3) (layers "F.Cu" "B.Cu") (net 9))
 (segment (start 36.6825 81.2561) (end 23.5881 81.2561) (width 0.25) (layer "B.Cu") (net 9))
 (segment (start 20.1881 86.1417) (end 18.1792 86.1417) (width 0.25) (layer "F.Cu") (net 5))
 (segment (start 20.8155 78.8923) (end 20.8155 78.2281) (width 0.25) (layer "F.Cu") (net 5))
 (segment (start 17.3525 84.787) (end 17.251 84.6855) (width 0.25) (layer "F.Cu") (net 5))
 (segment (start 7.2259 83.5092) (end 7.2259 84.6855) (width 0.25) (layer "F.Cu") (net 5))
 (segment (start 17.251 84.6855) (end 17.251 77.9041) (width 0.25) (layer "F.Cu") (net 5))
 (segment (start 21.5455 87.6227) (end 21.5455 87.4991) (width 0.25) (layer "F.Cu") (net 5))
 (segment (start 18.1792 84.915) (end 17.3525 84.915) (width 0.25) (layer "F.Cu") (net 5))
 (segment (start 18.1792 84.915) (end 18.1792 86.1417) (width 0.25) (layer "F.Cu") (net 5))
 (segment (start 20.7546 78.2281) (end 20.8155 78.2281) (width 0.25) (layer "F.Cu") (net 5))
 (segment (start 20.4306 77.9041) (end 20.7546 78.2281) (width 0.25) (layer "F.Cu") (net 5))
 (segment (start 17.3525 84.915) (end 17.3525 84.787) (width 0.25) (layer "F.Cu") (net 5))
 (segment (start 17.251 84.6855) (end 17.1495 84.6855) (width 0.25) (layer "F.Cu") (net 5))
 (segment (start 21.5455 87.4991) (end 20.1881 86.1417) (width 0.25) (layer "F.Cu") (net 5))
 (via (at 20.4306 77.9041) (size 0.6) (drill 0.3) (layers "F.Cu" "B.Cu") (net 5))
 (via (at 7.2259 84.6855) (size 0.6) (drill 0.3) (layers "F.Cu" "B.Cu") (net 5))
 (via (at 17.251 77.9041) (size 0.6) (drill 0.3) (layers "F.Cu" "B.Cu") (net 5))
 (via (at 17.1495 84.6855) (size 0.6) (drill 0.3) (layers "F.Cu" "B.Cu") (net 5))
 (segment (start 20.4306 77.9041) (end 17.251 77.9041) (width 0.25) (layer "B.Cu") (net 5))
 (segment (start 7.2259 84.6855) (end 17.1495 84.6855) (width 0.25) (layer "B.Cu") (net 5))
 (segment (start 19.0138 84.0763) (end 19.0138 81.8573) (width 0.25) (layer "F.Cu") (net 1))
 (segment (start 21.3155 79.5565) (end 21.9287 79.5565) (width 0.25) (layer "F.Cu") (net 1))
 (segment (start 19.8525 84.915) (end 19.0138 84.0763) (width 0.25) (layer "F.Cu") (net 1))
 (segment (start 21.9287 79.5565) (end 22.9273 80.5551) (width 0.25) (layer "F.Cu") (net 1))
 (segment (start 21.3155 78.8923) (end 21.3155 79.5565) (width 0.25) (layer "F.Cu") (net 1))
 (segment (start 22.0655 72.9148) (end 27.3578 78.2071) (width 0.25) (layer "F.Cu") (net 1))
 (segment (start 8.0009 78.3753) (end 8.0009 79.4166) (width 0.25) (layer "F.Cu") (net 1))
 (segment (start 27.3578 78.2071) (end 27.3578 78.7462) (width 0.25) (layer "F.Cu") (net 1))
 (segment (start 20.6792 84.915) (end 19.8525 84.915) (width 0.25) (layer "F.Cu") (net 1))
 (via (at 8.0009 79.4166) (size 0.6) (drill 0.3) (layers "F.Cu" "B.Cu") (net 1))
 (via (at 27.3578 78.7462) (size 0.6) (drill 0.3) (layers "F.Cu" "B.Cu") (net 1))
 (via (at 19.0138 81.8573) (size 0.6) (drill 0.3) (layers "F.Cu" "B.Cu") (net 1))
 (via (at 22.9273 80.5551) (size 0.6) (drill 0.3) (layers "F.Cu" "B.Cu") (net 1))
 (segment (start 25.5489 80.5551) (end 22.9273 80.5551) (width 0.25) (layer "B.Cu") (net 1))
 (segment (start 19.2042 80.5551) (end 19.0138 80.7455) (width 0.25) (layer "B.Cu") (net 1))
 (segment (start 22.9273 80.5551) (end 19.2042 80.5551) (width 0.25) (layer "B.Cu") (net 1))
 (segment (start 19.0138 80.7455) (end 19.0138 81.8573) (width 0.25) (layer "B.Cu") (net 1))
 (segment (start 9.3298 80.7455) (end 8.0009 79.4166) (width 0.25) (layer "B.Cu") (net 1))
 (segment (start 19.0138 80.7455) (end 9.3298 80.7455) (width 0.25) (layer "B.Cu") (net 1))
 (segment (start 27.3578 78.7462) (end 25.5489 80.5551) (width 0.25) (layer "B.Cu") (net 1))
 (segment (start 30.304 83.8843) (end 30.304 87.6767) (width 0.25) (layer "F.Cu") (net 7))
 (segment (start 23.0195 76.5998) (end 30.304 83.8843) (width 0.25) (layer "F.Cu") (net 7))
 (segment (start 21.2304 81.5531) (end 21.0385 81.3612) (width 0.25) (layer "F.Cu") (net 7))
 (segment (start 21.3155 82.2173) (end 21.3155 81.5531) (width 0.25) (layer "F.Cu") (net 7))
 (segment (start 22.0655 76.5998) (end 23.0195 76.5998) (width 0.25) (layer "F.Cu") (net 7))
 (segment (start 21.3155 81.5531) (end 21.2304 81.5531) (width 0.25) (layer "F.Cu") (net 7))
 (via (at 21.0385 81.3612) (size 0.6) (drill 0.3) (layers "F.Cu" "B.Cu") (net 7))
 (via (at 30.304 87.6767) (size 0.6) (drill 0.3) (layers "F.Cu" "B.Cu") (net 7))
 (segment (start 21.0385 81.746) (end 21.0385 81.3612) (width 0.25) (layer "B.Cu") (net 7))
 (segment (start 30.304 87.6767) (end 26.9692 87.6767) (width 0.25) (layer "B.Cu") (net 7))
 (segment (start 26.9692 87.6767) (end 21.0385 81.746) (width 0.25) (layer "B.Cu") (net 7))
 (segment (start 18.3142 89.0453) (end 16.6376 90.7219) (width 0.5) (layer "F.Cu") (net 2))
 (segment (start 21.332 74.3163) (end 22.0655 75.0498) (width 0.5) (layer "F.Cu") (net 2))
 (segment (start 5.5526 80.2859) (end 5.5526 79.2736) (width 0.5) (layer "F.Cu") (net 2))
 (segment (start 34.3621 87.0838) (end 34.3621 97.7594) (width 0.5) (layer "F.Cu") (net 2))
 (segment (start 21.8155 78.0067) (end 21.8155 78.8923) (width 0.2538) (layer "F.Cu") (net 2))
 (segment (start 19.1887 72.4294) (end 21.1148 72.4294) (width 0.5) (layer "F.Cu") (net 2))
 (segment (start 33.745 97.7594) (end 33.745 101.6716) (width 0.5) (layer "F.Cu") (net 2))
 (segment (start 10.0714 82.2137) (end 10.0714 80.708) (width 0.5) (layer "F.Cu") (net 2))
 (segment (start 19.1628 89.0453) (end 18.3142 89.0453) (width 0.5) (layer "F.Cu") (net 2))
 (segment (start 19.8155 83.0067) (end 21.0644 83.0067) (width 0.5) (layer "F.Cu") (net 2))
 (segment (start 8.7759 83.5092) (end 10.0714 82.2137) (width 0.5) (layer "F.Cu") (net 2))
 (segment (start 10.0792 82.2137) (end 10.0714 82.2137) (width 0.5) (layer "F.Cu") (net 2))
 (segment (start 29.9055 95.0372) (end 32.6277 97.7594) (width 0.5) (layer "F.Cu") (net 2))
 (segment (start 5.5239 80.2859) (end 5.255 80.5548) (width 0.5) (layer "F.Cu") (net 2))
 (segment (start 21.0644 83.0067) (end 23.4412 85.3835) (width 0.5) (layer "F.Cu") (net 2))
 (segment (start 19.1887 78.8546) (end 19.1887 72.4294) (width 0.5) (layer "F.Cu") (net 2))
 (segment (start 8.0009 76.8253) (end 11.0803 76.8253) (width 0.5) (layer "F.Cu") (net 2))
 (segment (start 15.7658 72.1398) (end 18.8991 72.1398) (width 0.5) (layer "F.Cu") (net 2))
 (segment (start 16.2105 88.345) (end 16.2105 90.2948) (width 0.5) (layer "F.Cu") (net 2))
 (segment (start 19.1629 89.0454) (end 19.1629 92.3179) (width 0.5) (layer "F.Cu") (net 2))
 (segment (start 32.6277 97.7594) (end 33.745 97.7594) (width 0.5) (layer "F.Cu") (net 2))
 (segment (start 19.9882 94.3082) (end 19.9882 97.4851) (width 0.5) (layer "F.Cu") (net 2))
 (segment (start 22.0655 75.0498) (end 22.3281 75.0498) (width 0.5) (layer "F.Cu") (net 2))
 (segment (start 19.678 81.3048) (end 19.8155 81.4423) (width 0.2538) (layer "F.Cu") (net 2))
 (segment (start 25.6954 88.4431) (end 24.1922 86.9399) (width 0.5) (layer "F.Cu") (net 2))
 (segment (start 16.2105 90.2948) (end 16.6376 90.7219) (width 0.5) (layer "F.Cu") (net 2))
 (segment (start 23.4412 85.3835) (end 23.4412 86.9399) (width 0.5) (layer "F.Cu") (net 2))
 (segment (start 21.1148 77.306) (end 21.1148 72.4294) (width 0.5) (layer "F.Cu") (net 2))
 (segment (start 8.7759 83.5092) (end 5.5526 80.2859) (width 0.5) (layer "F.Cu") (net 2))
 (segment (start 22.0655 71.9548) (end 21.8066 71.9548) (width 0.5) (layer "F.Cu") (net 2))
 (segment (start 19.1629 89.0453) (end 19.1628 89.0453) (width 0.5) (layer "F.Cu") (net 2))
 (segment (start 11.0803 76.8253) (end 15.7658 72.1398) (width 0.5) (layer "F.Cu") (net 2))
 (segment (start 5.5526 80.2859) (end 5.5239 80.2859) (width 0.5) (layer "F.Cu") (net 2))
 (segment (start 20.5855 87.6227) (end 19.1629 89.0453) (width 0.5) (layer "F.Cu") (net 2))
 (segment (start 21.1148 72.4294) (end 21.332 72.4294) (width 0.5) (layer "F.Cu") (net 2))
 (segment (start 19.1887 79.3155) (end 19.678 79.8048) (width 0.2538) (layer "F.Cu") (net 2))
 (segment (start 21.1288 88.4203) (end 20.5855 87.877) (width 0.5) (layer "F.Cu") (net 2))
 (segment (start 18.8991 72.1398) (end 19.1887 72.4294) (width 0.5) (layer "F.Cu") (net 2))
 (segment (start 5.5526 79.2736) (end 8.0009 76.8253) (width 0.5) (layer "F.Cu") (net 2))
 (segment (start 20.5855 87.877) (end 20.5855 87.6227) (width 0.5) (layer "F.Cu") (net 2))
 (segment (start 21.9608 88.4203) (end 21.1288 88.4203) (width 0.5) (layer "F.Cu") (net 2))
 (segment (start 24.1922 86.9399) (end 23.4412 86.9399) (width 0.5) (layer "F.Cu") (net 2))
 (segment (start 21.8066 71.9548) (end 21.332 72.4294) (width 0.5) (layer "F.Cu") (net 2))
 (segment (start 33.745 97.7594) (end 34.3621 97.7594) (width 0.5) (layer "F.Cu") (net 2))
 (segment (start 21.8155 78.0067) (end 21.1148 77.306) (width 0.5) (layer "F.Cu") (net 2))
 (segment (start 19.1887 78.8546) (end 19.1887 79.3155) (width 0.2538) (layer "F.Cu") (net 2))
 (segment (start 19.9882 97.4851) (end 19.043 98.4303) (width 0.5) (layer "F.Cu") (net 2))
 (segment (start 23.4412 86.9399) (end 21.9608 88.4203) (width 0.5) (layer "F.Cu") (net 2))
 (segment (start 16.2105 88.345) (end 10.0792 82.2137) (width 0.5) (layer "F.Cu") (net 2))
 (segment (start 19.8155 83.0067) (end 19.8155 82.8834) (width 0.2538) (layer "F.Cu") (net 2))
 (segment (start 19.8155 82.2173) (end 19.8155 82.8834) (width 0.2538) (layer "F.Cu") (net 2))
 (segment (start 19.8155 81.4423) (end 19.8155 82.2173) (width 0.2538) (layer "F.Cu") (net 2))
 (segment (start 21.332 72.4294) (end 21.332 74.3163) (width 0.5) (layer "F.Cu") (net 2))
 (segment (start 19.1629 89.0453) (end 19.1629 89.0454) (width 0.5) (layer "F.Cu") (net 2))
 (segment (start 22.3281 75.0498) (end 34.3621 87.0838) (width 0.5) (layer "F.Cu") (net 2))
 (segment (start 18.5804 92.9004) (end 19.9882 94.3082) (width 0.5) (layer "F.Cu") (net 2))
 (segment (start 19.1629 92.3179) (end 18.5804 92.9004) (width 0.5) (layer "F.Cu") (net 2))
 (segment (start 17.9628 99.3588) (end 21.8146 99.3588) (width 0.5) (layer "F.Cu") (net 3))
 (segment (start 24.1274 101.6716) (end 21.8146 99.3588) (width 0.5) (layer "F.Cu") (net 3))
 (segment (start 21.8146 99.3588) (end 21.8146 94.9539) (width 0.5) (layer "F.Cu") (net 3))
 (segment (start 14.3105 89.8773) (end 16.083 91.6498) (width 0.5) (layer "F.Cu") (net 3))
 (segment (start 17.2273 91.6498) (end 17.2273 98.6233) (width 0.5) (layer "F.Cu") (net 3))
 (segment (start 16.083 91.6498) (end 17.2273 91.6498) (width 0.5) (layer "F.Cu") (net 3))
 (segment (start 14.3105 88.345) (end 14.3105 89.8773) (width 0.5) (layer "F.Cu") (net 3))
 (segment (start 28.665 101.6716) (end 24.1274 101.6716) (width 0.5) (layer "F.Cu") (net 3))
 (segment (start 17.2273 98.6233) (end 17.9628 99.3588) (width 0.5) (layer "F.Cu") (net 3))
 (segment (start 17.2597 91.6498) (end 18.1876 90.7219) (width 0.5) (layer "F.Cu") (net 3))
 (segment (start 17.2273 91.6498) (end 17.2597 91.6498) (width 0.5) (layer "F.Cu") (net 3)))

